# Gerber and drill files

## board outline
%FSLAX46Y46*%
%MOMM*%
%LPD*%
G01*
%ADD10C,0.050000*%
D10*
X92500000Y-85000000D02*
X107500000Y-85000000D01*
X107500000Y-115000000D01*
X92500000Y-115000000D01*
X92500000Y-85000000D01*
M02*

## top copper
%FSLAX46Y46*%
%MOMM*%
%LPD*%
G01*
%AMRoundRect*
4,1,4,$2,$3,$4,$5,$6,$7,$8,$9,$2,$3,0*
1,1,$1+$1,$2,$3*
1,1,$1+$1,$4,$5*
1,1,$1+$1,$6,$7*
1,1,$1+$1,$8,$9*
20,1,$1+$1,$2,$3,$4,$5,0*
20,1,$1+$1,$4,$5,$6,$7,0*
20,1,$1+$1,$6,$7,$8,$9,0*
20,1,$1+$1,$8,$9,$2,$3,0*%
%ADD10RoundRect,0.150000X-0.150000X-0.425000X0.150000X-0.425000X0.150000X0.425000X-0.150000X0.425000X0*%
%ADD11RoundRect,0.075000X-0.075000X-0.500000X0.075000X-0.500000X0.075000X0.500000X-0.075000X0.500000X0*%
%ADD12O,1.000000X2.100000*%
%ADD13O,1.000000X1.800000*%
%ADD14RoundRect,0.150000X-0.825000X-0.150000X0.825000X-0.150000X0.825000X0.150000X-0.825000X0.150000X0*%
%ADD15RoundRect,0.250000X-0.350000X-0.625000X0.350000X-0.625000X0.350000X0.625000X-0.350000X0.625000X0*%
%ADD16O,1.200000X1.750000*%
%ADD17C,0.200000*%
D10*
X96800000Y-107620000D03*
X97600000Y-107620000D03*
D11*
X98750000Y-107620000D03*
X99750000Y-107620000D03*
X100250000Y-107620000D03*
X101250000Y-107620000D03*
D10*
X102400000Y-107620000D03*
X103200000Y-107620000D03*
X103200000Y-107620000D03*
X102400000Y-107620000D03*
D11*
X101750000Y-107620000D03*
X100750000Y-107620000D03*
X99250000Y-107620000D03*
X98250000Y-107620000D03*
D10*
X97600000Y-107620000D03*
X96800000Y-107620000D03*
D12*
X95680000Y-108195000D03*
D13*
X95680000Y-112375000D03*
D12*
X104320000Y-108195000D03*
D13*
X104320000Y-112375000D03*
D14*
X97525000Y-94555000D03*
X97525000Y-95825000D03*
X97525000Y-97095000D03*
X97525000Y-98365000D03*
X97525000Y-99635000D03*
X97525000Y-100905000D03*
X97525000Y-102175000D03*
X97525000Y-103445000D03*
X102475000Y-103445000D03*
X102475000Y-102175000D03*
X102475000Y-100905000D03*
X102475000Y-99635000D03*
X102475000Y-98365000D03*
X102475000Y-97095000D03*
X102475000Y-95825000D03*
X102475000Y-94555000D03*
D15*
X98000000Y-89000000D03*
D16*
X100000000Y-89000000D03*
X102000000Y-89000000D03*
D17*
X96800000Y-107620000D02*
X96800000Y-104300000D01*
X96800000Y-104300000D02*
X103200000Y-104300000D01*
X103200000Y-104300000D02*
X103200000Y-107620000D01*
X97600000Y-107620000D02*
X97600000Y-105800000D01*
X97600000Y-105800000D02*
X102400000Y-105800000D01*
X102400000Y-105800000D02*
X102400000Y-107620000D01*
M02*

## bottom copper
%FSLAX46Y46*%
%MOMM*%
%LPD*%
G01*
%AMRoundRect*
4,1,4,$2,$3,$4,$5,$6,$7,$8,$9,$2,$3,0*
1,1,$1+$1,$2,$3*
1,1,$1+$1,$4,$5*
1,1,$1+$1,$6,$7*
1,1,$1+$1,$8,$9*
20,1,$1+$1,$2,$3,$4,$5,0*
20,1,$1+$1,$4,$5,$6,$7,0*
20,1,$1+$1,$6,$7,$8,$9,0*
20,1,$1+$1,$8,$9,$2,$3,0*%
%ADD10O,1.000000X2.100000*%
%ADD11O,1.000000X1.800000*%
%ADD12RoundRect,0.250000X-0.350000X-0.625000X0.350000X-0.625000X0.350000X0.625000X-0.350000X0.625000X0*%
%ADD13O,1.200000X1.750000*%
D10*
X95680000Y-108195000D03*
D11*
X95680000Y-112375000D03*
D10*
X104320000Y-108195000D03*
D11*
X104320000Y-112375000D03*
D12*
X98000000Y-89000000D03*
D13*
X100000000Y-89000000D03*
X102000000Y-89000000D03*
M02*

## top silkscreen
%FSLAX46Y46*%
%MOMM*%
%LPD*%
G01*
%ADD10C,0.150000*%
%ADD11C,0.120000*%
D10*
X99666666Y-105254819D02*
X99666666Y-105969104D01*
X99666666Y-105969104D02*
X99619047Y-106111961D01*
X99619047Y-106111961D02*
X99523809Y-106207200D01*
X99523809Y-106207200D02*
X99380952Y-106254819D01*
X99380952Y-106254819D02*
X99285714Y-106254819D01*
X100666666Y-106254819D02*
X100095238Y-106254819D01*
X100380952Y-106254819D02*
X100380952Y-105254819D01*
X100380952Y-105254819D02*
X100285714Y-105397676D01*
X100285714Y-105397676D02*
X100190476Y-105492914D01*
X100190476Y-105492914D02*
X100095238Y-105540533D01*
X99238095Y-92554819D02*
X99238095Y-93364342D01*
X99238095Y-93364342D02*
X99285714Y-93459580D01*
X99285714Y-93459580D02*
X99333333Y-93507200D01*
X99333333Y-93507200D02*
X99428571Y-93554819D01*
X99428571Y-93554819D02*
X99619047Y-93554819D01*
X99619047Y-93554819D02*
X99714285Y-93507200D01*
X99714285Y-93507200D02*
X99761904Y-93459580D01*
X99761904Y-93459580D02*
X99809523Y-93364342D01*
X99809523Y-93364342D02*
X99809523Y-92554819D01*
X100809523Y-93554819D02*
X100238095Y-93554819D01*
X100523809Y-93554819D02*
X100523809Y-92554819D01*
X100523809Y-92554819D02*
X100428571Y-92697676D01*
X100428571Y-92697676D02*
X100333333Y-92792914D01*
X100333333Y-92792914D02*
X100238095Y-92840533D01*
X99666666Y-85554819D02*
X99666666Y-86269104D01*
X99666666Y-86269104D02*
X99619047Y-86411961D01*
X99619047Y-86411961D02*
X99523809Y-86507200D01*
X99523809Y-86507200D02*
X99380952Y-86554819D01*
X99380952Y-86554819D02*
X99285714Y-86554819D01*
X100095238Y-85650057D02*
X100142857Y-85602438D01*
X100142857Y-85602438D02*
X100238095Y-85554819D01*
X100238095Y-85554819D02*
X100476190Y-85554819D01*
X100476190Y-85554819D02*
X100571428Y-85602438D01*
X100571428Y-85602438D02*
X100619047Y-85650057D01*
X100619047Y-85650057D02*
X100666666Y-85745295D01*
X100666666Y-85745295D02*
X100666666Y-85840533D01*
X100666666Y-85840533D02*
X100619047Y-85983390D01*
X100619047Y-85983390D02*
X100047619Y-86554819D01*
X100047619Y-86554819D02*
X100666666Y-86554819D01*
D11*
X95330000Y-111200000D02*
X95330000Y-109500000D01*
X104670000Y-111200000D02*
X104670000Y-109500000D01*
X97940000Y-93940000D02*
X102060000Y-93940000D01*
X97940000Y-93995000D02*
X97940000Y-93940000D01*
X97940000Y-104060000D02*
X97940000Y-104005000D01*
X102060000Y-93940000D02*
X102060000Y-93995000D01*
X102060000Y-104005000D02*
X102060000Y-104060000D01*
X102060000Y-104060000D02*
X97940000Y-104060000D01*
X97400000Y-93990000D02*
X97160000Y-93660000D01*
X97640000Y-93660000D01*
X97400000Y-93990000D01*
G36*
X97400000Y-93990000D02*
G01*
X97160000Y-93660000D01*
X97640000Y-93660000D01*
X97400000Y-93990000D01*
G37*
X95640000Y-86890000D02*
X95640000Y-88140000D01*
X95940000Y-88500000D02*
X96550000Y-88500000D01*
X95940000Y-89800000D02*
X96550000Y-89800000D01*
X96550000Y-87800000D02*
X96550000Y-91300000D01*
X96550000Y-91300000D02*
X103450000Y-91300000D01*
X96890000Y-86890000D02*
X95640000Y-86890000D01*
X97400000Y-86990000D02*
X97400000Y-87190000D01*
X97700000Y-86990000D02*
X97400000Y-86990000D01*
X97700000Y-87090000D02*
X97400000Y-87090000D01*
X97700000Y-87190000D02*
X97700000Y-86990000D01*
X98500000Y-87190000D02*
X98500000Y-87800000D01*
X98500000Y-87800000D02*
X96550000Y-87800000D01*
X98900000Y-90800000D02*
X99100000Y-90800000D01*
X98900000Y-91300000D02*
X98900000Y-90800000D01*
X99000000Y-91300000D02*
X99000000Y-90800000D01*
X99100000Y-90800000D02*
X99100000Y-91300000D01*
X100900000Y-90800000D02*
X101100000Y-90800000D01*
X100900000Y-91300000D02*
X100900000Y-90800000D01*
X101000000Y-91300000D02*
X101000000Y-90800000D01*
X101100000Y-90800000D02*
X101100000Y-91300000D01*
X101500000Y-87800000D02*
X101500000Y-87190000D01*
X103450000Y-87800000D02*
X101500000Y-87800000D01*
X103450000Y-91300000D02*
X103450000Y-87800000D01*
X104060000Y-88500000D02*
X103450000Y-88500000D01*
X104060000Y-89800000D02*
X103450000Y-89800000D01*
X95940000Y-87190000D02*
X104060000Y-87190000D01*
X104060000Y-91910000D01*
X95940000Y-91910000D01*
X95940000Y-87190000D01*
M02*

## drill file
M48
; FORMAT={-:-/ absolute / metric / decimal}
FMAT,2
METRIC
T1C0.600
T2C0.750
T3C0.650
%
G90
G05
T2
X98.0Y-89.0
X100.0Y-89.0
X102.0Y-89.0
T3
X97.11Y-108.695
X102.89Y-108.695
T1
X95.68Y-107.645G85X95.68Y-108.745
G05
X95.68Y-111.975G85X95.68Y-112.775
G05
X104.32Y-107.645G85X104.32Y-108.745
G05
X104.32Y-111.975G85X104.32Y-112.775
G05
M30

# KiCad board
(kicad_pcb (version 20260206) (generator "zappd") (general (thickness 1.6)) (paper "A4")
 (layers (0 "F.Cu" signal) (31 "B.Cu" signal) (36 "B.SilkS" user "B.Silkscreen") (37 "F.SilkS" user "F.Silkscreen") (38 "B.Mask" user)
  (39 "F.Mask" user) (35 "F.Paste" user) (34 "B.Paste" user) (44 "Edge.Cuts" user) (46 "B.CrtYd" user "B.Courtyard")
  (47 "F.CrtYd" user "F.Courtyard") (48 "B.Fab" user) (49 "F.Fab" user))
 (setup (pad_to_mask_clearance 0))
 (gr_rect (start 92.5 85.0) (end 107.5 115.0) (stroke (width 0.05) (type default)) (fill none) (layer "Edge.Cuts"))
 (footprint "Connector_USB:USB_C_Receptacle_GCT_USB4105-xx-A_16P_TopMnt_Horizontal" (layer "F.Cu") (at 100 111.3)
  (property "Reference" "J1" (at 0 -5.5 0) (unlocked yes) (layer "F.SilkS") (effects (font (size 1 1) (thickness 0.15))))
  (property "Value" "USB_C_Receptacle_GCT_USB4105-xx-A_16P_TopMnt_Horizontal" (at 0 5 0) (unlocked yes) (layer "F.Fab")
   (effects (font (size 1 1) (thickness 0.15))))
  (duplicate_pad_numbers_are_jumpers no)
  (fp_line (start -4.67 -0.1) (end -4.67 -1.8) (stroke (width 0.12) (type solid)) (layer "F.SilkS"))
  (fp_line (start 4.67 -0.1) (end 4.67 -1.8) (stroke (width 0.12) (type solid)) (layer "F.SilkS"))
  (pad "" np_thru_hole circle (at -2.89 -2.605) (size 0.65 0.65) (drill 0.65) (layers "*.Cu" "*.Mask"))
  (pad "" np_thru_hole circle (at 2.89 -2.605) (size 0.65 0.65) (drill 0.65) (layers "*.Cu" "*.Mask"))
  (pad "A1" smd roundrect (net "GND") (at -3.2 -3.68) (size 0.6 1.15) (layers "F.Cu" "F.Mask" "F.Paste") (roundrect_rratio 0.25))
  (pad "A4" smd roundrect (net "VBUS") (at -2.4 -3.68) (size 0.6 1.15) (layers "F.Cu" "F.Mask" "F.Paste") (roundrect_rratio 0.25))
  (pad "A5" smd roundrect (at -1.25 -3.68) (size 0.3 1.15) (layers "F.Cu" "F.Mask" "F.Paste") (roundrect_rratio 0.25))
  (pad "A6" smd roundrect (at -0.25 -3.68) (size 0.3 1.15) (layers "F.Cu" "F.Mask" "F.Paste") (roundrect_rratio 0.25))
  (pad "A7" smd roundrect (at 0.25 -3.68) (size 0.3 1.15) (layers "F.Cu" "F.Mask" "F.Paste") (roundrect_rratio 0.25))
  (pad "A8" smd roundrect (at 1.25 -3.68) (size 0.3 1.15) (layers "F.Cu" "F.Mask" "F.Paste") (roundrect_rratio 0.25))
  (pad "A9" smd roundrect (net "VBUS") (at 2.4 -3.68) (size 0.6 1.15) (layers "F.Cu" "F.Mask" "F.Paste") (roundrect_rratio 0.25))
  (pad "A12" smd roundrect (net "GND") (at 3.2 -3.68) (size 0.6 1.15) (layers "F.Cu" "F.Mask" "F.Paste") (roundrect_rratio 0.25))
  (pad "B1" smd roundrect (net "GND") (at 3.2 -3.68) (size 0.6 1.15) (layers "F.Cu" "F.Mask" "F.Paste") (roundrect_rratio 0.25))
  (pad "B4" smd roundrect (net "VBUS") (at 2.4 -3.68) (size 0.6 1.15) (layers "F.Cu" "F.Mask" "F.Paste") (roundrect_rratio 0.25))
  (pad "B5" smd roundrect (at 1.75 -3.68) (size 0.3 1.15) (layers "F.Cu" "F.Mask" "F.Paste") (roundrect_rratio 0.25))
  (pad "B6" smd roundrect (at 0.75 -3.68) (size 0.3 1.15) (layers "F.Cu" "F.Mask" "F.Paste") (roundrect_rratio 0.25))
  (pad "B7" smd roundrect (at -0.75 -3.68) (size 0.3 1.15) (layers "F.Cu" "F.Mask" "F.Paste") (roundrect_rratio 0.25))
  (pad "B8" smd roundrect (at -1.75 -3.68) (size 0.3 1.15) (layers "F.Cu" "F.Mask" "F.Paste") (roundrect_rratio 0.25))
  (pad "B9" smd roundrect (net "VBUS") (at -2.4 -3.68) (size 0.6 1.15) (layers "F.Cu" "F.Mask" "F.Paste") (roundrect_rratio 0.25))
  (pad "B12" smd roundrect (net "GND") (at -3.2 -3.68) (size 0.6 1.15) (layers "F.Cu" "F.Mask" "F.Paste") (roundrect_rratio 0.25))
  (pad "SH" thru_hole oval (at -4.32 -3.105) (size 1 2.1) (drill oval 0.6 1.7) (layers "*.Cu" "*.Mask" "F.Paste") (remove_unused_layers no))
  (pad "SH" thru_hole oval (at -4.32 1.075) (size 1 1.8) (drill oval 0.6 1.4) (layers "*.Cu" "*.Mask" "F.Paste") (remove_unused_layers no))
  (pad "SH" thru_hole oval (at 4.32 -3.105) (size 1 2.1) (drill oval 0.6 1.7) (layers "*.Cu" "*.Mask" "F.Paste") (remove_unused_layers no))
  (pad "SH" thru_hole oval (at 4.32 1.075) (size 1 1.8) (drill oval 0.6 1.4) (layers "*.Cu" "*.Mask" "F.Paste") (remove_unused_layers no)))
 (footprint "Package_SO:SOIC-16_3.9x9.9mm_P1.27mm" (layer "F.Cu") (at 100 99)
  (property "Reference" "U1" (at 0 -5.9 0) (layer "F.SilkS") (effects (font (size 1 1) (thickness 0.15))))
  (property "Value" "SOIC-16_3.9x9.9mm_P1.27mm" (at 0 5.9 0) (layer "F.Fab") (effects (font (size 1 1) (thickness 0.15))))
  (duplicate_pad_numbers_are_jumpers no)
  (fp_line (start -2.06 -5.06) (end 2.06 -5.06) (stroke (width 0.12) (type solid)) (layer "F.SilkS"))
  (fp_line (start -2.06 -5.005) (end -2.06 -5.06) (stroke (width 0.12) (type solid)) (layer "F.SilkS"))
  (fp_line (start -2.06 5.06) (end -2.06 5.005) (stroke (width 0.12) (type solid)) (layer "F.SilkS"))
  (fp_line (start 2.06 -5.06) (end 2.06 -5.005) (stroke (width 0.12) (type solid)) (layer "F.SilkS"))
  (fp_line (start 2.06 5.005) (end 2.06 5.06) (stroke (width 0.12) (type solid)) (layer "F.SilkS"))
  (fp_line (start 2.06 5.06) (end -2.06 5.06) (stroke (width 0.12) (type solid)) (layer "F.SilkS"))
  (fp_poly (pts (xy -2.6 -5.01) (xy -2.84 -5.34) (xy -2.36 -5.34)) (stroke (width 0.12) (type solid)) (fill yes) (layer "F.SilkS"))
  (pad "1" smd roundrect (at -2.475 -4.445) (size 1.95 0.6) (layers "F.Cu" "F.Mask" "F.Paste") (roundrect_rratio 0.25))
  (pad "2" smd roundrect (at -2.475 -3.175) (size 1.95 0.6) (layers "F.Cu" "F.Mask" "F.Paste") (roundrect_rratio 0.25))
  (pad "3" smd roundrect (at -2.475 -1.905) (size 1.95 0.6) (layers "F.Cu" "F.Mask" "F.Paste") (roundrect_rratio 0.25))
  (pad "4" smd roundrect (at -2.475 -0.635) (size 1.95 0.6) (layers "F.Cu" "F.Mask" "F.Paste") (roundrect_rratio 0.25))
  (pad "5" smd roundrect (at -2.475 0.635) (size 1.95 0.6) (layers "F.Cu" "F.Mask" "F.Paste") (roundrect_rratio 0.25))
  (pad "6" smd roundrect (at -2.475 1.905) (size 1.95 0.6) (layers "F.Cu" "F.Mask" "F.Paste") (roundrect_rratio 0.25))
  (pad "7" smd roundrect (at -2.475 3.175) (size 1.95 0.6) (layers "F.Cu" "F.Mask" "F.Paste") (roundrect_rratio 0.25))
  (pad "8" smd roundrect (at -2.475 4.445) (size 1.95 0.6) (layers "F.Cu" "F.Mask" "F.Paste") (roundrect_rratio 0.25))
  (pad "9" smd roundrect (at 2.475 4.445) (size 1.95 0.6) (layers "F.Cu" "F.Mask" "F.Paste") (roundrect_rratio 0.25))
  (pad "10" smd roundrect (at 2.475 3.175) (size 1.95 0.6) (layers "F.Cu" "F.Mask" "F.Paste") (roundrect_rratio 0.25))
  (pad "11" smd roundrect (at 2.475 1.905) (size 1.95 0.6) (layers "F.Cu" "F.Mask" "F.Paste") (roundrect_rratio 0.25))
  (pad "12" smd roundrect (at 2.475 0.635) (size 1.95 0.6) (layers "F.Cu" "F.Mask" "F.Paste") (roundrect_rratio 0.25))
  (pad "13" smd roundrect (at 2.475 -0.635) (size 1.95 0.6) (layers "F.Cu" "F.Mask" "F.Paste") (roundrect_rratio 0.25))
  (pad "14" smd roundrect (at 2.475 -1.905) (size 1.95 0.6) (layers "F.Cu" "F.Mask" "F.Paste") (roundrect_rratio 0.25))
  (pad "15" smd roundrect (at 2.475 -3.175) (size 1.95 0.6) (layers "F.Cu" "F.Mask" "F.Paste") (roundrect_rratio 0.25))
  (pad "16" smd roundrect (at 2.475 -4.445) (size 1.95 0.6) (layers "F.Cu" "F.Mask" "F.Paste") (roundrect_rratio 0.25)))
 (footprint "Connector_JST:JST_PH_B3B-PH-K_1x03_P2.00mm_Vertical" (layer "F.Cu") (at 98 89)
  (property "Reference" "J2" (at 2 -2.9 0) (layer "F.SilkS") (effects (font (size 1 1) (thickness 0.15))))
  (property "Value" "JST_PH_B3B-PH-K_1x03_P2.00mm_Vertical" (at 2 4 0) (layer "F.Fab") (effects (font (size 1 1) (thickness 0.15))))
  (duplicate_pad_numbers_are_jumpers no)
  (fp_line (start -2.36 -2.11) (end -2.36 -0.86) (stroke (width 0.12) (type solid)) (layer "F.SilkS"))
  (fp_line (start -2.06 -0.5) (end -1.45 -0.5) (stroke (width 0.12) (type solid)) (layer "F.SilkS"))
  (fp_line (start -2.06 0.8) (end -1.45 0.8) (stroke (width 0.12) (type solid)) (layer "F.SilkS"))
  (fp_line (start -1.45 -1.2) (end -1.45 2.3) (stroke (width 0.12) (type solid)) (layer "F.SilkS"))
  (fp_line (start -1.45 2.3) (end 5.45 2.3) (stroke (width 0.12) (type solid)) (layer "F.SilkS"))
  (fp_line (start -1.11 -2.11) (end -2.36 -2.11) (stroke (width 0.12) (type solid)) (layer "F.SilkS"))
  (fp_line (start -0.6 -2.01) (end -0.6 -1.81) (stroke (width 0.12) (type solid)) (layer "F.SilkS"))
  (fp_line (start -0.3 -2.01) (end -0.6 -2.01) (stroke (width 0.12) (type solid)) (layer "F.SilkS"))
  (fp_line (start -0.3 -1.91) (end -0.6 -1.91) (stroke (width 0.12) (type solid)) (layer "F.SilkS"))
  (fp_line (start -0.3 -1.81) (end -0.3 -2.01) (stroke (width 0.12) (type solid)) (layer "F.SilkS"))
  (fp_line (start 0.5 -1.81) (end 0.5 -1.2) (stroke (width 0.12) (type solid)) (layer "F.SilkS"))
  (fp_line (start 0.5 -1.2) (end -1.45 -1.2) (stroke (width 0.12) (type solid)) (layer "F.SilkS"))
  (fp_line (start 0.9 1.8) (end 1.1 1.8) (stroke (width 0.12) (type solid)) (layer "F.SilkS"))
  (fp_line (start 0.9 2.3) (end 0.9 1.8) (stroke (width 0.12) (type solid)) (layer "F.SilkS"))
  (fp_line (start 1 2.3) (end 1 1.8) (stroke (width 0.12) (type solid)) (layer "F.SilkS"))
  (fp_line (start 1.1 1.8) (end 1.1 2.3) (stroke (width 0.12) (type solid)) (layer "F.SilkS"))
  (fp_line (start 2.9 1.8) (end 3.1 1.8) (stroke (width 0.12) (type solid)) (layer "F.SilkS"))
  (fp_line (start 2.9 2.3) (end 2.9 1.8) (stroke (width 0.12) (type solid)) (layer "F.SilkS"))
  (fp_line (start 3 2.3) (end 3 1.8) (stroke (width 0.12) (type solid)) (layer "F.SilkS"))
  (fp_line (start 3.1 1.8) (end 3.1 2.3) (stroke (width 0.12) (type solid)) (layer "F.SilkS"))
  (fp_line (start 3.5 -1.2) (end 3.5 -1.81) (stroke (width 0.12) (type solid)) (layer "F.SilkS"))
  (fp_line (start 5.45 -1.2) (end 3.5 -1.2) (stroke (width 0.12) (type solid)) (layer "F.SilkS"))
  (fp_line (start 5.45 2.3) (end 5.45 -1.2) (stroke (width 0.12) (type solid)) (layer "F.SilkS"))
  (fp_line (start 6.06 -0.5) (end 5.45 -0.5) (stroke (width 0.12) (type solid)) (layer "F.SilkS"))
  (fp_line (start 6.06 0.8) (end 5.45 0.8) (stroke (width 0.12) (type solid)) (layer "F.SilkS"))
  (fp_rect (start -2.06 -1.81) (end 6.06 2.91) (stroke (width 0.12) (type solid)) (fill no) (layer "F.SilkS"))
  (pad "1" thru_hole roundrect (at 0 0) (size 1.2 1.75) (drill 0.75) (layers "*.Cu" "*.Mask") (remove_unused_layers no)
   (roundrect_rratio 0.208333))
  (pad "2" thru_hole oval (at 2 0) (size 1.2 1.75) (drill 0.75) (layers "*.Cu" "*.Mask") (remove_unused_layers no))
  (pad "3" thru_hole oval (at 4 0) (size 1.2 1.75) (drill 0.75) (layers "*.Cu" "*.Mask") (remove_unused_layers no)))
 (segment (start 96.8000 107.6200) (end 96.8000 104.3000) (width 0.2) (layer "F.Cu") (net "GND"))
 (segment (start 96.8000 104.3000) (end 103.2000 104.3000) (width 0.2) (layer "F.Cu") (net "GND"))
 (segment (start 103.2000 104.3000) (end 103.2000 107.6200) (width 0.2) (layer "F.Cu") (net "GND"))
 (segment (start 97.6000 107.6200) (end 97.6000 105.8000) (width 0.2) (layer "F.Cu") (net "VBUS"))
 (segment (start 97.6000 105.8000) (end 102.4000 105.8000) (width 0.2) (layer "F.Cu") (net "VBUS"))
 (segment (start 102.4000 105.8000) (end 102.4000 107.6200) (width 0.2) (layer "F.Cu") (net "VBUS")))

